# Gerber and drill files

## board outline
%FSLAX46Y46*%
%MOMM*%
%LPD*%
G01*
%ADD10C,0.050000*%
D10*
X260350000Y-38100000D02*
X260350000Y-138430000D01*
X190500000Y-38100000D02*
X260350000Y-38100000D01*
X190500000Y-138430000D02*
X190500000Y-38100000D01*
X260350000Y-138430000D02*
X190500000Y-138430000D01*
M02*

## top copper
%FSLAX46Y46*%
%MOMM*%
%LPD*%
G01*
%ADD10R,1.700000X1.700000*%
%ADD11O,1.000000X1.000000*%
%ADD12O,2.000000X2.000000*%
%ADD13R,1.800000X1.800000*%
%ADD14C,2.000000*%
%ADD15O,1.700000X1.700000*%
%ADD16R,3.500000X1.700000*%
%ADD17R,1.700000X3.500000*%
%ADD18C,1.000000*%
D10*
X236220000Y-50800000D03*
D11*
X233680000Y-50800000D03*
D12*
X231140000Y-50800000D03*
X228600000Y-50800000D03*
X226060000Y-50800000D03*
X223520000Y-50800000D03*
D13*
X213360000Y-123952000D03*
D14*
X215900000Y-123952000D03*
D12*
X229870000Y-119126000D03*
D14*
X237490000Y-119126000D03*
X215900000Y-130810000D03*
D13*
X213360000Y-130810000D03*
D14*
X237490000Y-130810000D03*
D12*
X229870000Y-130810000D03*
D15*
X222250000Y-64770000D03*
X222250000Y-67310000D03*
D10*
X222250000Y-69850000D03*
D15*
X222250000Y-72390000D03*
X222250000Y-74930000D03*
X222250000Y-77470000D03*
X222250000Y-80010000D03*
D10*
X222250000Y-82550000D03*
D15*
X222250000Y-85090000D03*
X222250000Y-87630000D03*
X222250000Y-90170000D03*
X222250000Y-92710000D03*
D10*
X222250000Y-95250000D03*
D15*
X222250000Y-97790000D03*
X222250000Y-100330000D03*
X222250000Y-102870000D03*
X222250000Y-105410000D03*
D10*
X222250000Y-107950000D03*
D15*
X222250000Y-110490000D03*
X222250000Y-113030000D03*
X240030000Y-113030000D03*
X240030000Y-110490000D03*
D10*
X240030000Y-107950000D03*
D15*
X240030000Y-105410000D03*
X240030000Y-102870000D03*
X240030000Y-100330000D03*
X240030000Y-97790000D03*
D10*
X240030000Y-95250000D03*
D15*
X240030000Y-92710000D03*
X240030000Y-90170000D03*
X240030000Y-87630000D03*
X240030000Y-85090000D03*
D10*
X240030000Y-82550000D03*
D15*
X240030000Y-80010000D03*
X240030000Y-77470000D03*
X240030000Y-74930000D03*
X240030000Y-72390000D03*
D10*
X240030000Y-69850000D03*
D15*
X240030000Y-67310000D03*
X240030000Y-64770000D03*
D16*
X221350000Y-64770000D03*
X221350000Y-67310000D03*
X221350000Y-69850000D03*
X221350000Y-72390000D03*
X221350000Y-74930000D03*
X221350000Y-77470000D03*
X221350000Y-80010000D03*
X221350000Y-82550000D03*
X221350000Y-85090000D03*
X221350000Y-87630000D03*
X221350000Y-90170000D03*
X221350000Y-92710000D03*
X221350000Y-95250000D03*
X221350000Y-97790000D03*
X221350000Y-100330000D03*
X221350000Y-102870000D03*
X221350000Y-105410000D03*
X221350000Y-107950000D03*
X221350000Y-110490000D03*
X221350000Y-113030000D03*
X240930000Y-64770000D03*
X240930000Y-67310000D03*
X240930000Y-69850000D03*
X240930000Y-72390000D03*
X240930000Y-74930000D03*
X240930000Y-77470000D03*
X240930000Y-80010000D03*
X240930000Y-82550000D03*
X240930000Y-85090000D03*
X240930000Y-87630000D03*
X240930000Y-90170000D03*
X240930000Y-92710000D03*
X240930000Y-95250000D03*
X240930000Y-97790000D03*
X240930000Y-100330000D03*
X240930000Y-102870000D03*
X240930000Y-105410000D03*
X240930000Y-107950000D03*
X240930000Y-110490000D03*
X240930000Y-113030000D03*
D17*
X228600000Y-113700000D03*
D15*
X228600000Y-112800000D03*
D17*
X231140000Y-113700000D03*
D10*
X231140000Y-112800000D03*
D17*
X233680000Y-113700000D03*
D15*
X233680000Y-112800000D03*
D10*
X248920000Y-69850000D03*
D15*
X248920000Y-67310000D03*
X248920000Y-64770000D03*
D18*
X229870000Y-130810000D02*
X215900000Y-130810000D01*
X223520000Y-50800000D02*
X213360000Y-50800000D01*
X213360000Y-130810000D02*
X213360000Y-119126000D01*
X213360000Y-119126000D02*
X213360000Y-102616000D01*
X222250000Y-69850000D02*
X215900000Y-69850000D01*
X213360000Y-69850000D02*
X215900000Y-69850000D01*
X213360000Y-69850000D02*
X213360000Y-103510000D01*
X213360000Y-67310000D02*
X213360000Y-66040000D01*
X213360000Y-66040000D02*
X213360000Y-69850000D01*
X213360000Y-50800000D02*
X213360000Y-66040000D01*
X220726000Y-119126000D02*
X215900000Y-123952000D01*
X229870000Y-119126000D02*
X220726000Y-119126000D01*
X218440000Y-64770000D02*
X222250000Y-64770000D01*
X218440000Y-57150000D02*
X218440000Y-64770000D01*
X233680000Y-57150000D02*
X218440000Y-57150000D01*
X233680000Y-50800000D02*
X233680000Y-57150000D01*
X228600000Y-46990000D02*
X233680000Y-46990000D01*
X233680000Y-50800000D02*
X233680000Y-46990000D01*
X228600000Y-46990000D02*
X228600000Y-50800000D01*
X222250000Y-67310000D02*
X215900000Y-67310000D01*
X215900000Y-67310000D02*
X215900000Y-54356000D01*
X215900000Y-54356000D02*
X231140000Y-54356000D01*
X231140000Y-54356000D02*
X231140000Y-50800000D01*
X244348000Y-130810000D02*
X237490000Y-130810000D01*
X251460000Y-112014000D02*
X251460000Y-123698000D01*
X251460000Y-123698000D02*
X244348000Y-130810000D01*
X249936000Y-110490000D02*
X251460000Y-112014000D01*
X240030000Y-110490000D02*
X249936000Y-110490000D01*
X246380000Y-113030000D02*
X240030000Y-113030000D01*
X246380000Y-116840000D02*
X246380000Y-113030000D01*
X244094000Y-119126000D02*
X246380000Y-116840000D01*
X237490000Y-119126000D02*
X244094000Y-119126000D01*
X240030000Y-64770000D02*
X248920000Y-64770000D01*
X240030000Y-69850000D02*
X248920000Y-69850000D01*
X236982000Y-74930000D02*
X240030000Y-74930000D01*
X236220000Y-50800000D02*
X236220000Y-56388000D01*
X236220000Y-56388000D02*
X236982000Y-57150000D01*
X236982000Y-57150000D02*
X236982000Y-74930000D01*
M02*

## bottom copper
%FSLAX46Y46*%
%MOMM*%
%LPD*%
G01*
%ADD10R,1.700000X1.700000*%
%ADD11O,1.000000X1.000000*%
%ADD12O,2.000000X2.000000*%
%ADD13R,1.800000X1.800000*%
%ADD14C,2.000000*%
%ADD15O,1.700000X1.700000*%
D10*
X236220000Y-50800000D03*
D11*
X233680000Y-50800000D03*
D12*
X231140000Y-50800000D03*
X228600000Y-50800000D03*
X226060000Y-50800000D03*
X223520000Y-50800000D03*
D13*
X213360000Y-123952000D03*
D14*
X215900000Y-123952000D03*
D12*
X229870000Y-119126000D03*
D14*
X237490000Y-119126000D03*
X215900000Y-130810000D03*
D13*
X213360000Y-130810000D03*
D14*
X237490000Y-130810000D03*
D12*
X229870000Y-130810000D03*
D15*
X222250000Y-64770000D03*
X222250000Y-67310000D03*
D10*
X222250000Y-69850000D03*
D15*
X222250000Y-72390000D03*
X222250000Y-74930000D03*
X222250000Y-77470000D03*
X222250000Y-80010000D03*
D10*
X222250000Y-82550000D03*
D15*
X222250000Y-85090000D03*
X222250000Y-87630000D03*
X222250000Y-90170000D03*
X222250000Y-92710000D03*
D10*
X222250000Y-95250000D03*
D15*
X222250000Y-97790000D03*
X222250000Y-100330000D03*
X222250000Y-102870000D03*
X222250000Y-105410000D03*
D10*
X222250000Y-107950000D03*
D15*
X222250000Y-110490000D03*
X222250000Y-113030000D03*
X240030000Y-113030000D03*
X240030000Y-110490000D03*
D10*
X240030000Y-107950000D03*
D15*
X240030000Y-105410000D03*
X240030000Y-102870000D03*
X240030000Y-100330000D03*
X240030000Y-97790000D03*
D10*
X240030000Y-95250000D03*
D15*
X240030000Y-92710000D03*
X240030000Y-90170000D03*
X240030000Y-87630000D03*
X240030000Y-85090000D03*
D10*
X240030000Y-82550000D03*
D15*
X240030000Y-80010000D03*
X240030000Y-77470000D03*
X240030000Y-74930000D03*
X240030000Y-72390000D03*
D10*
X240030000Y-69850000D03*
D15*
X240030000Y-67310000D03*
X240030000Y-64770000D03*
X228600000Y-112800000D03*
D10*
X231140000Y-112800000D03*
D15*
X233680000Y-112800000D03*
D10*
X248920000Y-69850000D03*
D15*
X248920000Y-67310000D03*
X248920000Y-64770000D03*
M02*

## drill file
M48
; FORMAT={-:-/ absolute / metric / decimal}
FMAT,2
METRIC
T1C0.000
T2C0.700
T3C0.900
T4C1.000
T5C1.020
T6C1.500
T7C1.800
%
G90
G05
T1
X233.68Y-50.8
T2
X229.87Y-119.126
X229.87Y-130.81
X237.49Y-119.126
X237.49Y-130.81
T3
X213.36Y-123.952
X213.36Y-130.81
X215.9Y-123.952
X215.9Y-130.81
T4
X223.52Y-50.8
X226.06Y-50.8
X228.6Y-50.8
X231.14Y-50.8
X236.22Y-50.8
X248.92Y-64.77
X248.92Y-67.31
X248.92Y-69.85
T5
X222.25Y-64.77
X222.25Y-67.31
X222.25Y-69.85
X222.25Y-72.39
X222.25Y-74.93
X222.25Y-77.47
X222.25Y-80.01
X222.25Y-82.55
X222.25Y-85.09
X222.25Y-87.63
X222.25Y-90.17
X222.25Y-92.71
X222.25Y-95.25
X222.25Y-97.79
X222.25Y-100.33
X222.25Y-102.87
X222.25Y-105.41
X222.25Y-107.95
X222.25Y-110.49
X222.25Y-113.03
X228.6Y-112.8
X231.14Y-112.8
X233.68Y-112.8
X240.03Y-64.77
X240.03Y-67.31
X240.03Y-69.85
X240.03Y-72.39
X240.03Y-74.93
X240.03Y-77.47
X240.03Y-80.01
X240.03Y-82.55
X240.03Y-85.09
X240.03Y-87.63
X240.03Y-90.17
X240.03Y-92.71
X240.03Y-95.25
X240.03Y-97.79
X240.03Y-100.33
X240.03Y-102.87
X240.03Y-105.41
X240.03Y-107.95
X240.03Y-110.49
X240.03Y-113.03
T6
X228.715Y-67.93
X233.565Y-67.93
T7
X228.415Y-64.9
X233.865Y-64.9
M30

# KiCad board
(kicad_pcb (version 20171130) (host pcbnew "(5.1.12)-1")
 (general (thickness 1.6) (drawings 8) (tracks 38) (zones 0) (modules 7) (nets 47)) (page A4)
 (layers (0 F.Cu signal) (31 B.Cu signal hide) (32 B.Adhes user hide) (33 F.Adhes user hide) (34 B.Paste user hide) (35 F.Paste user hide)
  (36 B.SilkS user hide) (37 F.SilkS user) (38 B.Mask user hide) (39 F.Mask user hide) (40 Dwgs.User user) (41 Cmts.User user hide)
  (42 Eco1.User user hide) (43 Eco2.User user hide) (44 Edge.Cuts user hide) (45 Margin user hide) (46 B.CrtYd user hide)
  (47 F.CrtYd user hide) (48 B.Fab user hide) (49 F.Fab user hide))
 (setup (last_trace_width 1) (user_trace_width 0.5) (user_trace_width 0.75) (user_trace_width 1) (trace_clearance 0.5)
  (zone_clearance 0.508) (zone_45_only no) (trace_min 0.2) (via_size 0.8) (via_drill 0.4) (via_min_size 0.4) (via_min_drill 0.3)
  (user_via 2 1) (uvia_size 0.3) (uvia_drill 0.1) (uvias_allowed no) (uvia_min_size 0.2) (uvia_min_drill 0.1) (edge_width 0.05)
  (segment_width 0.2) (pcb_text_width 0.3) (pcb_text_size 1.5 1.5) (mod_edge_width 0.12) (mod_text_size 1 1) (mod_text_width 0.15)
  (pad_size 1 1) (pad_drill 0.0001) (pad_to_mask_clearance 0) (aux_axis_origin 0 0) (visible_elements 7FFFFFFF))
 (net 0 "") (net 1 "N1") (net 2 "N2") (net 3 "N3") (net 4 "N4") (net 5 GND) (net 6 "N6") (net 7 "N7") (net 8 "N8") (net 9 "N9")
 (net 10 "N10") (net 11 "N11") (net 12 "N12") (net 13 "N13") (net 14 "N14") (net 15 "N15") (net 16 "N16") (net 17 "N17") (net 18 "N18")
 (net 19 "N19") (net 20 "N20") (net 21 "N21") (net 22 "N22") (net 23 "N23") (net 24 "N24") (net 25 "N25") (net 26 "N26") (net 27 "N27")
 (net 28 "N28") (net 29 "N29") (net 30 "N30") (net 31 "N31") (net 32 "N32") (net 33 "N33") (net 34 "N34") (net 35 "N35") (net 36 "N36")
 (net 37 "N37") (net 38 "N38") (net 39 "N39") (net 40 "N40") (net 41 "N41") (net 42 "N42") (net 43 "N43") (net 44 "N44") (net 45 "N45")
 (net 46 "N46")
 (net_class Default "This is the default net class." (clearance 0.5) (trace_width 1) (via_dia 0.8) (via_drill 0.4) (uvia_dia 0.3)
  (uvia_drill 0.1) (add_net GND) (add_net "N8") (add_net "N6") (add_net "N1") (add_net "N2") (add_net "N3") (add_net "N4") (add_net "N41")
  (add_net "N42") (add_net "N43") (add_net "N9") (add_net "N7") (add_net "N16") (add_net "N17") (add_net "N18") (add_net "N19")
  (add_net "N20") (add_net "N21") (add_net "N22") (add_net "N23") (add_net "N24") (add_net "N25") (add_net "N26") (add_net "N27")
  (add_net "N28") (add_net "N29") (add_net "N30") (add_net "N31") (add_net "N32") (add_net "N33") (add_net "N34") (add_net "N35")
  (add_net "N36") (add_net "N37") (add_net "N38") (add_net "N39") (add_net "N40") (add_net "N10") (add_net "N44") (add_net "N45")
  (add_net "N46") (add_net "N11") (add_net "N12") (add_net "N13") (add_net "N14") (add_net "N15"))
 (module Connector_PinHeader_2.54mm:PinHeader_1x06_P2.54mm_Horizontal (layer F.Cu) (at 236.22 50.8 270)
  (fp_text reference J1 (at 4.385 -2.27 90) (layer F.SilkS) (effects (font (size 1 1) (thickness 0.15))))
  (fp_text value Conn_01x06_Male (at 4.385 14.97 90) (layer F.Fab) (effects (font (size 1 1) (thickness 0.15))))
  (pad 1 thru_hole rect (at 0 0 270) (size 1.7 1.7) (drill 1) (layers *.Cu *.Mask) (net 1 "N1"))
  (pad 2 thru_hole oval (at 0 2.54 270) (size 1 1) (drill 0.0001) (layers *.Cu *.Mask) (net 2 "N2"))
  (pad 3 thru_hole oval (at 0 5.08 270) (size 2 2) (drill 1) (layers *.Cu *.Mask) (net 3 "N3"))
  (pad 4 thru_hole oval (at 0 7.62 270) (size 2 2) (drill 1) (layers *.Cu *.Mask) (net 2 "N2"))
  (pad 5 thru_hole oval (at 0 10.16 270) (size 2 2) (drill 1) (layers *.Cu *.Mask) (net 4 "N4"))
  (pad 6 thru_hole oval (at 0 12.7 270) (size 2 2) (drill 1) (layers *.Cu *.Mask) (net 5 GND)))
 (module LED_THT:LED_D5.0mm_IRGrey (layer F.Cu) (at 213.36 123.952)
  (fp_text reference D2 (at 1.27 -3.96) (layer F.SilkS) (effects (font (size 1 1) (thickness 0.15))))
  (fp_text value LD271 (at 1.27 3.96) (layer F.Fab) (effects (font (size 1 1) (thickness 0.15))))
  (pad 1 thru_hole rect (at 0 0) (size 1.8 1.8) (drill 0.9) (layers *.Cu *.Mask) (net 5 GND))
  (pad 2 thru_hole circle (at 2.54 0) (size 2 2) (drill 0.9) (layers *.Cu *.Mask) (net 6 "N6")))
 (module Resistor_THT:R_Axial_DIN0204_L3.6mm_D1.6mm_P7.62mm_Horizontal (layer F.Cu) (at 237.49 119.126 180)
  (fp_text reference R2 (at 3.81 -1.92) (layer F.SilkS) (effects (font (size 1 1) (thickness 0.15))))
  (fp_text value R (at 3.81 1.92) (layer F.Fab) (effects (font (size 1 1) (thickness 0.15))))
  (pad 2 thru_hole oval (at 7.62 0 180) (size 2 2) (drill 0.7) (layers *.Cu *.Mask) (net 6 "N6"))
  (pad 1 thru_hole circle (at 0 0 180) (size 2 2) (drill 0.7) (layers *.Cu *.Mask) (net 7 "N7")))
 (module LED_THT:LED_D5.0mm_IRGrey (layer F.Cu) (at 213.36 130.81)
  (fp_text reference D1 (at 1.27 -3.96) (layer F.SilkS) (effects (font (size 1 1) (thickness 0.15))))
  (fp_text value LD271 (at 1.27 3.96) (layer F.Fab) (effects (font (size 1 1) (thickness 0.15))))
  (pad 2 thru_hole circle (at 2.54 0) (size 2 2) (drill 0.9) (layers *.Cu *.Mask) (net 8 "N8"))
  (pad 1 thru_hole rect (at 0 0) (size 1.8 1.8) (drill 0.9) (layers *.Cu *.Mask) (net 5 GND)))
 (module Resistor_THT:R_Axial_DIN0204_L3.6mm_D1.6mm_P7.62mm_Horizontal (layer F.Cu) (at 237.49 130.81 180)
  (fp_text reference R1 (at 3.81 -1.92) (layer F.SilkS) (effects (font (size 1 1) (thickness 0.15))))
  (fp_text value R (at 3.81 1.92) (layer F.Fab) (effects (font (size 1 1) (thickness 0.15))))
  (pad 1 thru_hole circle (at 0 0 180) (size 2 2) (drill 0.7) (layers *.Cu *.Mask) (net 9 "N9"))
  (pad 2 thru_hole oval (at 7.62 0 180) (size 2 2) (drill 0.7) (layers *.Cu *.Mask) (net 8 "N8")))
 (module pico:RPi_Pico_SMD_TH (layer F.Cu) (at 231.14 88.9)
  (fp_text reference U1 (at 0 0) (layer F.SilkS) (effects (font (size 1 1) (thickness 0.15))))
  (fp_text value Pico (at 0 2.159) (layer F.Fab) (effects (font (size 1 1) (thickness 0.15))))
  (pad 1 thru_hole oval (at -8.89 -24.13) (size 1.7 1.7) (drill 1.02) (layers *.Cu *.Mask) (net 2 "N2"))
  (pad 2 thru_hole oval (at -8.89 -21.59) (size 1.7 1.7) (drill 1.02) (layers *.Cu *.Mask) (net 3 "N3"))
  (pad 3 thru_hole rect (at -8.89 -19.05) (size 1.7 1.7) (drill 1.02) (layers *.Cu *.Mask) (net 5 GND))
  (pad 4 thru_hole oval (at -8.89 -16.51) (size 1.7 1.7) (drill 1.02) (layers *.Cu *.Mask) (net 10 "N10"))
  (pad 5 thru_hole oval (at -8.89 -13.97) (size 1.7 1.7) (drill 1.02) (layers *.Cu *.Mask) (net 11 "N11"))
  (pad 6 thru_hole oval (at -8.89 -11.43) (size 1.7 1.7) (drill 1.02) (layers *.Cu *.Mask) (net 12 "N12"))
  (pad 7 thru_hole oval (at -8.89 -8.89) (size 1.7 1.7) (drill 1.02) (layers *.Cu *.Mask) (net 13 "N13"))
  (pad 8 thru_hole rect (at -8.89 -6.35) (size 1.7 1.7) (drill 1.02) (layers *.Cu *.Mask) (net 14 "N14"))
  (pad 9 thru_hole oval (at -8.89 -3.81) (size 1.7 1.7) (drill 1.02) (layers *.Cu *.Mask) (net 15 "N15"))
  (pad 10 thru_hole oval (at -8.89 -1.27) (size 1.7 1.7) (drill 1.02) (layers *.Cu *.Mask) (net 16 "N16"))
  (pad 11 thru_hole oval (at -8.89 1.27) (size 1.7 1.7) (drill 1.02) (layers *.Cu *.Mask) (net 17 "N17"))
  (pad 12 thru_hole oval (at -8.89 3.81) (size 1.7 1.7) (drill 1.02) (layers *.Cu *.Mask) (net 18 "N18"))
  (pad 13 thru_hole rect (at -8.89 6.35) (size 1.7 1.7) (drill 1.02) (layers *.Cu *.Mask) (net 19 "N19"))
  (pad 14 thru_hole oval (at -8.89 8.89) (size 1.7 1.7) (drill 1.02) (layers *.Cu *.Mask) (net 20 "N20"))
  (pad 15 thru_hole oval (at -8.89 11.43) (size 1.7 1.7) (drill 1.02) (layers *.Cu *.Mask) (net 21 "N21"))
  (pad 16 thru_hole oval (at -8.89 13.97) (size 1.7 1.7) (drill 1.02) (layers *.Cu *.Mask) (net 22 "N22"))
  (pad 17 thru_hole oval (at -8.89 16.51) (size 1.7 1.7) (drill 1.02) (layers *.Cu *.Mask) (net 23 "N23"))
  (pad 18 thru_hole rect (at -8.89 19.05) (size 1.7 1.7) (drill 1.02) (layers *.Cu *.Mask) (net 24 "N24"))
  (pad 19 thru_hole oval (at -8.89 21.59) (size 1.7 1.7) (drill 1.02) (layers *.Cu *.Mask) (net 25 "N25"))
  (pad 20 thru_hole oval (at -8.89 24.13) (size 1.7 1.7) (drill 1.02) (layers *.Cu *.Mask) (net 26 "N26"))
  (pad 21 thru_hole oval (at 8.89 24.13) (size 1.7 1.7) (drill 1.02) (layers *.Cu *.Mask) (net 7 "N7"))
  (pad 22 thru_hole oval (at 8.89 21.59) (size 1.7 1.7) (drill 1.02) (layers *.Cu *.Mask) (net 9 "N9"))
  (pad 23 thru_hole rect (at 8.89 19.05) (size 1.7 1.7) (drill 1.02) (layers *.Cu *.Mask) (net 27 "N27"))
  (pad 24 thru_hole oval (at 8.89 16.51) (size 1.7 1.7) (drill 1.02) (layers *.Cu *.Mask) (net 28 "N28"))
  (pad 25 thru_hole oval (at 8.89 13.97) (size 1.7 1.7) (drill 1.02) (layers *.Cu *.Mask) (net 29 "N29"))
  (pad 26 thru_hole oval (at 8.89 11.43) (size 1.7 1.7) (drill 1.02) (layers *.Cu *.Mask) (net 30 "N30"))
  (pad 27 thru_hole oval (at 8.89 8.89) (size 1.7 1.7) (drill 1.02) (layers *.Cu *.Mask) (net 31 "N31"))
  (pad 28 thru_hole rect (at 8.89 6.35) (size 1.7 1.7) (drill 1.02) (layers *.Cu *.Mask) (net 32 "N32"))
  (pad 29 thru_hole oval (at 8.89 3.81) (size 1.7 1.7) (drill 1.02) (layers *.Cu *.Mask) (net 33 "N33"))
  (pad 30 thru_hole oval (at 8.89 1.27) (size 1.7 1.7) (drill 1.02) (layers *.Cu *.Mask) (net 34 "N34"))
  (pad 31 thru_hole oval (at 8.89 -1.27) (size 1.7 1.7) (drill 1.02) (layers *.Cu *.Mask) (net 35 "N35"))
  (pad 32 thru_hole oval (at 8.89 -3.81) (size 1.7 1.7) (drill 1.02) (layers *.Cu *.Mask) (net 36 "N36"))
  (pad 33 thru_hole rect (at 8.89 -6.35) (size 1.7 1.7) (drill 1.02) (layers *.Cu *.Mask) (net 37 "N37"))
  (pad 34 thru_hole oval (at 8.89 -8.89) (size 1.7 1.7) (drill 1.02) (layers *.Cu *.Mask) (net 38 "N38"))
  (pad 35 thru_hole oval (at 8.89 -11.43) (size 1.7 1.7) (drill 1.02) (layers *.Cu *.Mask) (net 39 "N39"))
  (pad 36 thru_hole oval (at 8.89 -13.97) (size 1.7 1.7) (drill 1.02) (layers *.Cu *.Mask) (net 1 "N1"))
  (pad 37 thru_hole oval (at 8.89 -16.51) (size 1.7 1.7) (drill 1.02) (layers *.Cu *.Mask) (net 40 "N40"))
  (pad 38 thru_hole rect (at 8.89 -19.05) (size 1.7 1.7) (drill 1.02) (layers *.Cu *.Mask) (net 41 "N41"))
  (pad 39 thru_hole oval (at 8.89 -21.59) (size 1.7 1.7) (drill 1.02) (layers *.Cu *.Mask) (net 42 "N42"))
  (pad 40 thru_hole oval (at 8.89 -24.13) (size 1.7 1.7) (drill 1.02) (layers *.Cu *.Mask) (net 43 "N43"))
  (pad 1 smd rect (at -8.89 -24.13) (size 3.5 1.7) (drill (offset -0.9 0)) (layers F.Cu F.Mask) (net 2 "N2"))
  (pad 2 smd rect (at -8.89 -21.59) (size 3.5 1.7) (drill (offset -0.9 0)) (layers F.Cu F.Mask) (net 3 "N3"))
  (pad 3 smd rect (at -8.89 -19.05) (size 3.5 1.7) (drill (offset -0.9 0)) (layers F.Cu F.Mask) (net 5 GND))
  (pad 4 smd rect (at -8.89 -16.51) (size 3.5 1.7) (drill (offset -0.9 0)) (layers F.Cu F.Mask) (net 10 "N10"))
  (pad 5 smd rect (at -8.89 -13.97) (size 3.5 1.7) (drill (offset -0.9 0)) (layers F.Cu F.Mask) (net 11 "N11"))
  (pad 6 smd rect (at -8.89 -11.43) (size 3.5 1.7) (drill (offset -0.9 0)) (layers F.Cu F.Mask) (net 12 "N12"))
  (pad 7 smd rect (at -8.89 -8.89) (size 3.5 1.7) (drill (offset -0.9 0)) (layers F.Cu F.Mask) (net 13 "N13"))
  (pad 8 smd rect (at -8.89 -6.35) (size 3.5 1.7) (drill (offset -0.9 0)) (layers F.Cu F.Mask) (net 14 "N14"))
  (pad 9 smd rect (at -8.89 -3.81) (size 3.5 1.7) (drill (offset -0.9 0)) (layers F.Cu F.Mask) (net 15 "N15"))
  (pad 10 smd rect (at -8.89 -1.27) (size 3.5 1.7) (drill (offset -0.9 0)) (layers F.Cu F.Mask) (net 16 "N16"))
  (pad 11 smd rect (at -8.89 1.27) (size 3.5 1.7) (drill (offset -0.9 0)) (layers F.Cu F.Mask) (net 17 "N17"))
  (pad 12 smd rect (at -8.89 3.81) (size 3.5 1.7) (drill (offset -0.9 0)) (layers F.Cu F.Mask) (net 18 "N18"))
  (pad 13 smd rect (at -8.89 6.35) (size 3.5 1.7) (drill (offset -0.9 0)) (layers F.Cu F.Mask) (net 19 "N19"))
  (pad 14 smd rect (at -8.89 8.89) (size 3.5 1.7) (drill (offset -0.9 0)) (layers F.Cu F.Mask) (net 20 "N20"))
  (pad 15 smd rect (at -8.89 11.43) (size 3.5 1.7) (drill (offset -0.9 0)) (layers F.Cu F.Mask) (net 21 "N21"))
  (pad 16 smd rect (at -8.89 13.97) (size 3.5 1.7) (drill (offset -0.9 0)) (layers F.Cu F.Mask) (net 22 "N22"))
  (pad 17 smd rect (at -8.89 16.51) (size 3.5 1.7) (drill (offset -0.9 0)) (layers F.Cu F.Mask) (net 23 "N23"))
  (pad 18 smd rect (at -8.89 19.05) (size 3.5 1.7) (drill (offset -0.9 0)) (layers F.Cu F.Mask) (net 24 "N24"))
  (pad 19 smd rect (at -8.89 21.59) (size 3.5 1.7) (drill (offset -0.9 0)) (layers F.Cu F.Mask) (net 25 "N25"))
  (pad 20 smd rect (at -8.89 24.13) (size 3.5 1.7) (drill (offset -0.9 0)) (layers F.Cu F.Mask) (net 26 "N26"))
  (pad 40 smd rect (at 8.89 -24.13) (size 3.5 1.7) (drill (offset 0.9 0)) (layers F.Cu F.Mask) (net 43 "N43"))
  (pad 39 smd rect (at 8.89 -21.59) (size 3.5 1.7) (drill (offset 0.9 0)) (layers F.Cu F.Mask) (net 42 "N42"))
  (pad 38 smd rect (at 8.89 -19.05) (size 3.5 1.7) (drill (offset 0.9 0)) (layers F.Cu F.Mask) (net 41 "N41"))
  (pad 37 smd rect (at 8.89 -16.51) (size 3.5 1.7) (drill (offset 0.9 0)) (layers F.Cu F.Mask) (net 40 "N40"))
  (pad 36 smd rect (at 8.89 -13.97) (size 3.5 1.7) (drill (offset 0.9 0)) (layers F.Cu F.Mask) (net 1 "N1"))
  (pad 35 smd rect (at 8.89 -11.43) (size 3.5 1.7) (drill (offset 0.9 0)) (layers F.Cu F.Mask) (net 39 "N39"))
  (pad 34 smd rect (at 8.89 -8.89) (size 3.5 1.7) (drill (offset 0.9 0)) (layers F.Cu F.Mask) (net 38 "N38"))
  (pad 33 smd rect (at 8.89 -6.35) (size 3.5 1.7) (drill (offset 0.9 0)) (layers F.Cu F.Mask) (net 37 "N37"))
  (pad 32 smd rect (at 8.89 -3.81) (size 3.5 1.7) (drill (offset 0.9 0)) (layers F.Cu F.Mask) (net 36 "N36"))
  (pad 31 smd rect (at 8.89 -1.27) (size 3.5 1.7) (drill (offset 0.9 0)) (layers F.Cu F.Mask) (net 35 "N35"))
  (pad 30 smd rect (at 8.89 1.27) (size 3.5 1.7) (drill (offset 0.9 0)) (layers F.Cu F.Mask) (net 34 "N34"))
  (pad 29 smd rect (at 8.89 3.81) (size 3.5 1.7) (drill (offset 0.9 0)) (layers F.Cu F.Mask) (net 33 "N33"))
  (pad 28 smd rect (at 8.89 6.35) (size 3.5 1.7) (drill (offset 0.9 0)) (layers F.Cu F.Mask) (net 32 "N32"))
  (pad 27 smd rect (at 8.89 8.89) (size 3.5 1.7) (drill (offset 0.9 0)) (layers F.Cu F.Mask) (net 31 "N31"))
  (pad 26 smd rect (at 8.89 11.43) (size 3.5 1.7) (drill (offset 0.9 0)) (layers F.Cu F.Mask) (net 30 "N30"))
  (pad 25 smd rect (at 8.89 13.97) (size 3.5 1.7) (drill (offset 0.9 0)) (layers F.Cu F.Mask) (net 29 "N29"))
  (pad 24 smd rect (at 8.89 16.51) (size 3.5 1.7) (drill (offset 0.9 0)) (layers F.Cu F.Mask) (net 28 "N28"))
  (pad 23 smd rect (at 8.89 19.05) (size 3.5 1.7) (drill (offset 0.9 0)) (layers F.Cu F.Mask) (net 27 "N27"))
  (pad 22 smd rect (at 8.89 21.59) (size 3.5 1.7) (drill (offset 0.9 0)) (layers F.Cu F.Mask) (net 9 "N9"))
  (pad 21 smd rect (at 8.89 24.13) (size 3.5 1.7) (drill (offset 0.9 0)) (layers F.Cu F.Mask) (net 7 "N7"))
  (pad "" np_thru_hole oval (at -2.725 -24) (size 1.8 1.8) (drill 1.8) (layers *.Cu *.Mask))
  (pad "" np_thru_hole oval (at 2.725 -24) (size 1.8 1.8) (drill 1.8) (layers *.Cu *.Mask))
  (pad "" np_thru_hole oval (at -2.425 -20.97) (size 1.5 1.5) (drill 1.5) (layers *.Cu *.Mask))
  (pad "" np_thru_hole oval (at 2.425 -20.97) (size 1.5 1.5) (drill 1.5) (layers *.Cu *.Mask))
  (pad 41 smd rect (at -2.54 23.9 90) (size 3.5 1.7) (drill (offset -0.9 0)) (layers F.Cu F.Mask) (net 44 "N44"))
  (pad 41 thru_hole oval (at -2.54 23.9) (size 1.7 1.7) (drill 1.02) (layers *.Cu *.Mask) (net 44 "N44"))
  (pad 42 smd rect (at 0 23.9 90) (size 3.5 1.7) (drill (offset -0.9 0)) (layers F.Cu F.Mask) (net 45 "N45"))
  (pad 42 thru_hole rect (at 0 23.9) (size 1.7 1.7) (drill 1.02) (layers *.Cu *.Mask) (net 45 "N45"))
  (pad 43 smd rect (at 2.54 23.9 90) (size 3.5 1.7) (drill (offset -0.9 0)) (layers F.Cu F.Mask) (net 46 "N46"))
  (pad 43 thru_hole oval (at 2.54 23.9) (size 1.7 1.7) (drill 1.02) (layers *.Cu *.Mask) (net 46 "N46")))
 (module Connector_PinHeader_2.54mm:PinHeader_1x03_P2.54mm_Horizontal (layer F.Cu) (at 248.92 69.85 180)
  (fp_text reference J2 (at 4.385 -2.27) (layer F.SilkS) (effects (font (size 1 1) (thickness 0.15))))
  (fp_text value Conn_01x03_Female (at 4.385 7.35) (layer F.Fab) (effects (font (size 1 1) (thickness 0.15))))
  (pad 1 thru_hole rect (at 0 0 180) (size 1.7 1.7) (drill 1) (layers *.Cu *.Mask) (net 41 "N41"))
  (pad 2 thru_hole oval (at 0 2.54 180) (size 1.7 1.7) (drill 1) (layers *.Cu *.Mask) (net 42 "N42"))
  (pad 3 thru_hole oval (at 0 5.08 180) (size 1.7 1.7) (drill 1) (layers *.Cu *.Mask) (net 43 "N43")))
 (gr_line (start 260.35 38.1) (end 260.35 138.43) (layer Edge.Cuts) (width 0.05))
 (gr_line (start 190.5 38.1) (end 260.35 38.1) (layer Edge.Cuts) (width 0.05))
 (gr_line (start 190.5 138.43) (end 190.5 38.1) (layer Edge.Cuts) (width 0.05))
 (gr_line (start 260.35 138.43) (end 190.5 138.43) (layer Edge.Cuts) (width 0.05))
 (segment (start 229.87 130.81) (end 215.9 130.81) (width 1) (layer F.Cu) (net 8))
 (segment (start 223.52 50.8) (end 213.36 50.8) (width 1) (layer F.Cu) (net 5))
 (segment (start 213.36 130.81) (end 213.36 119.126) (width 1) (layer F.Cu) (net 5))
 (segment (start 213.36 119.126) (end 213.36 102.616) (width 1) (layer F.Cu) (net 5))
 (segment (start 222.25 69.85) (end 215.9 69.85) (width 1) (layer F.Cu) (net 5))
 (segment (start 213.36 69.85) (end 215.9 69.85) (width 1) (layer F.Cu) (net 5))
 (segment (start 213.36 69.85) (end 213.36 103.51) (width 1) (layer F.Cu) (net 5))
 (segment (start 213.36 67.31) (end 213.36 66.04) (width 1) (layer F.Cu) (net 5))
 (segment (start 213.36 66.04) (end 213.36 69.85) (width 1) (layer F.Cu) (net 5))
 (segment (start 213.36 50.8) (end 213.36 66.04) (width 1) (layer F.Cu) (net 5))
 (segment (start 220.726 119.126) (end 215.9 123.952) (width 1) (layer F.Cu) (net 6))
 (segment (start 229.87 119.126) (end 220.726 119.126) (width 1) (layer F.Cu) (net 6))
 (segment (start 218.44 64.77) (end 222.25 64.77) (width 1) (layer F.Cu) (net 2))
 (segment (start 218.44 57.15) (end 218.44 64.77) (width 1) (layer F.Cu) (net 2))
 (segment (start 233.68 57.15) (end 218.44 57.15) (width 1) (layer F.Cu) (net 2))
 (segment (start 233.68 50.8) (end 233.68 57.15) (width 1) (layer F.Cu) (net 2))
 (segment (start 228.6 46.99) (end 233.68 46.99) (width 1) (layer F.Cu) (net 2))
 (segment (start 233.68 50.8) (end 233.68 46.99) (width 1) (layer F.Cu) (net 2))
 (segment (start 228.6 46.99) (end 228.6 50.8) (width 1) (layer F.Cu) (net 2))
 (segment (start 222.25 67.31) (end 215.9 67.31) (width 1) (layer F.Cu) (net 3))
 (segment (start 215.9 67.31) (end 215.9 54.356) (width 1) (layer F.Cu) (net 3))
 (segment (start 215.9 54.356) (end 231.14 54.356) (width 1) (layer F.Cu) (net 3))
 (segment (start 231.14 54.356) (end 231.14 50.8) (width 1) (layer F.Cu) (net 3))
 (segment (start 244.348 130.81) (end 237.49 130.81) (width 1) (layer F.Cu) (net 9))
 (segment (start 251.46 112.014) (end 251.46 123.698) (width 1) (layer F.Cu) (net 9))
 (segment (start 251.46 123.698) (end 244.348 130.81) (width 1) (layer F.Cu) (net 9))
 (segment (start 249.936 110.49) (end 251.46 112.014) (width 1) (layer F.Cu) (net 9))
 (segment (start 240.03 110.49) (end 249.936 110.49) (width 1) (layer F.Cu) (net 9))
 (segment (start 246.38 113.03) (end 240.03 113.03) (width 1) (layer F.Cu) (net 7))
 (segment (start 246.38 116.84) (end 246.38 113.03) (width 1) (layer F.Cu) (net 7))
 (segment (start 244.094 119.126) (end 246.38 116.84) (width 1) (layer F.Cu) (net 7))
 (segment (start 237.49 119.126) (end 244.094 119.126) (width 1) (layer F.Cu) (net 7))
 (segment (start 240.03 64.77) (end 248.92 64.77) (width 1) (layer F.Cu) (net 43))
 (segment (start 240.03 69.85) (end 248.92 69.85) (width 1) (layer F.Cu) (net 41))
 (segment (start 236.982 74.93) (end 240.03 74.93) (width 1) (layer F.Cu) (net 1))
 (segment (start 236.22 50.8) (end 236.22 56.388) (width 1) (layer F.Cu) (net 1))
 (segment (start 236.22 56.388) (end 236.982 57.15) (width 1) (layer F.Cu) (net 1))
 (segment (start 236.982 57.15) (end 236.982 74.93) (width 1) (layer F.Cu) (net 1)))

